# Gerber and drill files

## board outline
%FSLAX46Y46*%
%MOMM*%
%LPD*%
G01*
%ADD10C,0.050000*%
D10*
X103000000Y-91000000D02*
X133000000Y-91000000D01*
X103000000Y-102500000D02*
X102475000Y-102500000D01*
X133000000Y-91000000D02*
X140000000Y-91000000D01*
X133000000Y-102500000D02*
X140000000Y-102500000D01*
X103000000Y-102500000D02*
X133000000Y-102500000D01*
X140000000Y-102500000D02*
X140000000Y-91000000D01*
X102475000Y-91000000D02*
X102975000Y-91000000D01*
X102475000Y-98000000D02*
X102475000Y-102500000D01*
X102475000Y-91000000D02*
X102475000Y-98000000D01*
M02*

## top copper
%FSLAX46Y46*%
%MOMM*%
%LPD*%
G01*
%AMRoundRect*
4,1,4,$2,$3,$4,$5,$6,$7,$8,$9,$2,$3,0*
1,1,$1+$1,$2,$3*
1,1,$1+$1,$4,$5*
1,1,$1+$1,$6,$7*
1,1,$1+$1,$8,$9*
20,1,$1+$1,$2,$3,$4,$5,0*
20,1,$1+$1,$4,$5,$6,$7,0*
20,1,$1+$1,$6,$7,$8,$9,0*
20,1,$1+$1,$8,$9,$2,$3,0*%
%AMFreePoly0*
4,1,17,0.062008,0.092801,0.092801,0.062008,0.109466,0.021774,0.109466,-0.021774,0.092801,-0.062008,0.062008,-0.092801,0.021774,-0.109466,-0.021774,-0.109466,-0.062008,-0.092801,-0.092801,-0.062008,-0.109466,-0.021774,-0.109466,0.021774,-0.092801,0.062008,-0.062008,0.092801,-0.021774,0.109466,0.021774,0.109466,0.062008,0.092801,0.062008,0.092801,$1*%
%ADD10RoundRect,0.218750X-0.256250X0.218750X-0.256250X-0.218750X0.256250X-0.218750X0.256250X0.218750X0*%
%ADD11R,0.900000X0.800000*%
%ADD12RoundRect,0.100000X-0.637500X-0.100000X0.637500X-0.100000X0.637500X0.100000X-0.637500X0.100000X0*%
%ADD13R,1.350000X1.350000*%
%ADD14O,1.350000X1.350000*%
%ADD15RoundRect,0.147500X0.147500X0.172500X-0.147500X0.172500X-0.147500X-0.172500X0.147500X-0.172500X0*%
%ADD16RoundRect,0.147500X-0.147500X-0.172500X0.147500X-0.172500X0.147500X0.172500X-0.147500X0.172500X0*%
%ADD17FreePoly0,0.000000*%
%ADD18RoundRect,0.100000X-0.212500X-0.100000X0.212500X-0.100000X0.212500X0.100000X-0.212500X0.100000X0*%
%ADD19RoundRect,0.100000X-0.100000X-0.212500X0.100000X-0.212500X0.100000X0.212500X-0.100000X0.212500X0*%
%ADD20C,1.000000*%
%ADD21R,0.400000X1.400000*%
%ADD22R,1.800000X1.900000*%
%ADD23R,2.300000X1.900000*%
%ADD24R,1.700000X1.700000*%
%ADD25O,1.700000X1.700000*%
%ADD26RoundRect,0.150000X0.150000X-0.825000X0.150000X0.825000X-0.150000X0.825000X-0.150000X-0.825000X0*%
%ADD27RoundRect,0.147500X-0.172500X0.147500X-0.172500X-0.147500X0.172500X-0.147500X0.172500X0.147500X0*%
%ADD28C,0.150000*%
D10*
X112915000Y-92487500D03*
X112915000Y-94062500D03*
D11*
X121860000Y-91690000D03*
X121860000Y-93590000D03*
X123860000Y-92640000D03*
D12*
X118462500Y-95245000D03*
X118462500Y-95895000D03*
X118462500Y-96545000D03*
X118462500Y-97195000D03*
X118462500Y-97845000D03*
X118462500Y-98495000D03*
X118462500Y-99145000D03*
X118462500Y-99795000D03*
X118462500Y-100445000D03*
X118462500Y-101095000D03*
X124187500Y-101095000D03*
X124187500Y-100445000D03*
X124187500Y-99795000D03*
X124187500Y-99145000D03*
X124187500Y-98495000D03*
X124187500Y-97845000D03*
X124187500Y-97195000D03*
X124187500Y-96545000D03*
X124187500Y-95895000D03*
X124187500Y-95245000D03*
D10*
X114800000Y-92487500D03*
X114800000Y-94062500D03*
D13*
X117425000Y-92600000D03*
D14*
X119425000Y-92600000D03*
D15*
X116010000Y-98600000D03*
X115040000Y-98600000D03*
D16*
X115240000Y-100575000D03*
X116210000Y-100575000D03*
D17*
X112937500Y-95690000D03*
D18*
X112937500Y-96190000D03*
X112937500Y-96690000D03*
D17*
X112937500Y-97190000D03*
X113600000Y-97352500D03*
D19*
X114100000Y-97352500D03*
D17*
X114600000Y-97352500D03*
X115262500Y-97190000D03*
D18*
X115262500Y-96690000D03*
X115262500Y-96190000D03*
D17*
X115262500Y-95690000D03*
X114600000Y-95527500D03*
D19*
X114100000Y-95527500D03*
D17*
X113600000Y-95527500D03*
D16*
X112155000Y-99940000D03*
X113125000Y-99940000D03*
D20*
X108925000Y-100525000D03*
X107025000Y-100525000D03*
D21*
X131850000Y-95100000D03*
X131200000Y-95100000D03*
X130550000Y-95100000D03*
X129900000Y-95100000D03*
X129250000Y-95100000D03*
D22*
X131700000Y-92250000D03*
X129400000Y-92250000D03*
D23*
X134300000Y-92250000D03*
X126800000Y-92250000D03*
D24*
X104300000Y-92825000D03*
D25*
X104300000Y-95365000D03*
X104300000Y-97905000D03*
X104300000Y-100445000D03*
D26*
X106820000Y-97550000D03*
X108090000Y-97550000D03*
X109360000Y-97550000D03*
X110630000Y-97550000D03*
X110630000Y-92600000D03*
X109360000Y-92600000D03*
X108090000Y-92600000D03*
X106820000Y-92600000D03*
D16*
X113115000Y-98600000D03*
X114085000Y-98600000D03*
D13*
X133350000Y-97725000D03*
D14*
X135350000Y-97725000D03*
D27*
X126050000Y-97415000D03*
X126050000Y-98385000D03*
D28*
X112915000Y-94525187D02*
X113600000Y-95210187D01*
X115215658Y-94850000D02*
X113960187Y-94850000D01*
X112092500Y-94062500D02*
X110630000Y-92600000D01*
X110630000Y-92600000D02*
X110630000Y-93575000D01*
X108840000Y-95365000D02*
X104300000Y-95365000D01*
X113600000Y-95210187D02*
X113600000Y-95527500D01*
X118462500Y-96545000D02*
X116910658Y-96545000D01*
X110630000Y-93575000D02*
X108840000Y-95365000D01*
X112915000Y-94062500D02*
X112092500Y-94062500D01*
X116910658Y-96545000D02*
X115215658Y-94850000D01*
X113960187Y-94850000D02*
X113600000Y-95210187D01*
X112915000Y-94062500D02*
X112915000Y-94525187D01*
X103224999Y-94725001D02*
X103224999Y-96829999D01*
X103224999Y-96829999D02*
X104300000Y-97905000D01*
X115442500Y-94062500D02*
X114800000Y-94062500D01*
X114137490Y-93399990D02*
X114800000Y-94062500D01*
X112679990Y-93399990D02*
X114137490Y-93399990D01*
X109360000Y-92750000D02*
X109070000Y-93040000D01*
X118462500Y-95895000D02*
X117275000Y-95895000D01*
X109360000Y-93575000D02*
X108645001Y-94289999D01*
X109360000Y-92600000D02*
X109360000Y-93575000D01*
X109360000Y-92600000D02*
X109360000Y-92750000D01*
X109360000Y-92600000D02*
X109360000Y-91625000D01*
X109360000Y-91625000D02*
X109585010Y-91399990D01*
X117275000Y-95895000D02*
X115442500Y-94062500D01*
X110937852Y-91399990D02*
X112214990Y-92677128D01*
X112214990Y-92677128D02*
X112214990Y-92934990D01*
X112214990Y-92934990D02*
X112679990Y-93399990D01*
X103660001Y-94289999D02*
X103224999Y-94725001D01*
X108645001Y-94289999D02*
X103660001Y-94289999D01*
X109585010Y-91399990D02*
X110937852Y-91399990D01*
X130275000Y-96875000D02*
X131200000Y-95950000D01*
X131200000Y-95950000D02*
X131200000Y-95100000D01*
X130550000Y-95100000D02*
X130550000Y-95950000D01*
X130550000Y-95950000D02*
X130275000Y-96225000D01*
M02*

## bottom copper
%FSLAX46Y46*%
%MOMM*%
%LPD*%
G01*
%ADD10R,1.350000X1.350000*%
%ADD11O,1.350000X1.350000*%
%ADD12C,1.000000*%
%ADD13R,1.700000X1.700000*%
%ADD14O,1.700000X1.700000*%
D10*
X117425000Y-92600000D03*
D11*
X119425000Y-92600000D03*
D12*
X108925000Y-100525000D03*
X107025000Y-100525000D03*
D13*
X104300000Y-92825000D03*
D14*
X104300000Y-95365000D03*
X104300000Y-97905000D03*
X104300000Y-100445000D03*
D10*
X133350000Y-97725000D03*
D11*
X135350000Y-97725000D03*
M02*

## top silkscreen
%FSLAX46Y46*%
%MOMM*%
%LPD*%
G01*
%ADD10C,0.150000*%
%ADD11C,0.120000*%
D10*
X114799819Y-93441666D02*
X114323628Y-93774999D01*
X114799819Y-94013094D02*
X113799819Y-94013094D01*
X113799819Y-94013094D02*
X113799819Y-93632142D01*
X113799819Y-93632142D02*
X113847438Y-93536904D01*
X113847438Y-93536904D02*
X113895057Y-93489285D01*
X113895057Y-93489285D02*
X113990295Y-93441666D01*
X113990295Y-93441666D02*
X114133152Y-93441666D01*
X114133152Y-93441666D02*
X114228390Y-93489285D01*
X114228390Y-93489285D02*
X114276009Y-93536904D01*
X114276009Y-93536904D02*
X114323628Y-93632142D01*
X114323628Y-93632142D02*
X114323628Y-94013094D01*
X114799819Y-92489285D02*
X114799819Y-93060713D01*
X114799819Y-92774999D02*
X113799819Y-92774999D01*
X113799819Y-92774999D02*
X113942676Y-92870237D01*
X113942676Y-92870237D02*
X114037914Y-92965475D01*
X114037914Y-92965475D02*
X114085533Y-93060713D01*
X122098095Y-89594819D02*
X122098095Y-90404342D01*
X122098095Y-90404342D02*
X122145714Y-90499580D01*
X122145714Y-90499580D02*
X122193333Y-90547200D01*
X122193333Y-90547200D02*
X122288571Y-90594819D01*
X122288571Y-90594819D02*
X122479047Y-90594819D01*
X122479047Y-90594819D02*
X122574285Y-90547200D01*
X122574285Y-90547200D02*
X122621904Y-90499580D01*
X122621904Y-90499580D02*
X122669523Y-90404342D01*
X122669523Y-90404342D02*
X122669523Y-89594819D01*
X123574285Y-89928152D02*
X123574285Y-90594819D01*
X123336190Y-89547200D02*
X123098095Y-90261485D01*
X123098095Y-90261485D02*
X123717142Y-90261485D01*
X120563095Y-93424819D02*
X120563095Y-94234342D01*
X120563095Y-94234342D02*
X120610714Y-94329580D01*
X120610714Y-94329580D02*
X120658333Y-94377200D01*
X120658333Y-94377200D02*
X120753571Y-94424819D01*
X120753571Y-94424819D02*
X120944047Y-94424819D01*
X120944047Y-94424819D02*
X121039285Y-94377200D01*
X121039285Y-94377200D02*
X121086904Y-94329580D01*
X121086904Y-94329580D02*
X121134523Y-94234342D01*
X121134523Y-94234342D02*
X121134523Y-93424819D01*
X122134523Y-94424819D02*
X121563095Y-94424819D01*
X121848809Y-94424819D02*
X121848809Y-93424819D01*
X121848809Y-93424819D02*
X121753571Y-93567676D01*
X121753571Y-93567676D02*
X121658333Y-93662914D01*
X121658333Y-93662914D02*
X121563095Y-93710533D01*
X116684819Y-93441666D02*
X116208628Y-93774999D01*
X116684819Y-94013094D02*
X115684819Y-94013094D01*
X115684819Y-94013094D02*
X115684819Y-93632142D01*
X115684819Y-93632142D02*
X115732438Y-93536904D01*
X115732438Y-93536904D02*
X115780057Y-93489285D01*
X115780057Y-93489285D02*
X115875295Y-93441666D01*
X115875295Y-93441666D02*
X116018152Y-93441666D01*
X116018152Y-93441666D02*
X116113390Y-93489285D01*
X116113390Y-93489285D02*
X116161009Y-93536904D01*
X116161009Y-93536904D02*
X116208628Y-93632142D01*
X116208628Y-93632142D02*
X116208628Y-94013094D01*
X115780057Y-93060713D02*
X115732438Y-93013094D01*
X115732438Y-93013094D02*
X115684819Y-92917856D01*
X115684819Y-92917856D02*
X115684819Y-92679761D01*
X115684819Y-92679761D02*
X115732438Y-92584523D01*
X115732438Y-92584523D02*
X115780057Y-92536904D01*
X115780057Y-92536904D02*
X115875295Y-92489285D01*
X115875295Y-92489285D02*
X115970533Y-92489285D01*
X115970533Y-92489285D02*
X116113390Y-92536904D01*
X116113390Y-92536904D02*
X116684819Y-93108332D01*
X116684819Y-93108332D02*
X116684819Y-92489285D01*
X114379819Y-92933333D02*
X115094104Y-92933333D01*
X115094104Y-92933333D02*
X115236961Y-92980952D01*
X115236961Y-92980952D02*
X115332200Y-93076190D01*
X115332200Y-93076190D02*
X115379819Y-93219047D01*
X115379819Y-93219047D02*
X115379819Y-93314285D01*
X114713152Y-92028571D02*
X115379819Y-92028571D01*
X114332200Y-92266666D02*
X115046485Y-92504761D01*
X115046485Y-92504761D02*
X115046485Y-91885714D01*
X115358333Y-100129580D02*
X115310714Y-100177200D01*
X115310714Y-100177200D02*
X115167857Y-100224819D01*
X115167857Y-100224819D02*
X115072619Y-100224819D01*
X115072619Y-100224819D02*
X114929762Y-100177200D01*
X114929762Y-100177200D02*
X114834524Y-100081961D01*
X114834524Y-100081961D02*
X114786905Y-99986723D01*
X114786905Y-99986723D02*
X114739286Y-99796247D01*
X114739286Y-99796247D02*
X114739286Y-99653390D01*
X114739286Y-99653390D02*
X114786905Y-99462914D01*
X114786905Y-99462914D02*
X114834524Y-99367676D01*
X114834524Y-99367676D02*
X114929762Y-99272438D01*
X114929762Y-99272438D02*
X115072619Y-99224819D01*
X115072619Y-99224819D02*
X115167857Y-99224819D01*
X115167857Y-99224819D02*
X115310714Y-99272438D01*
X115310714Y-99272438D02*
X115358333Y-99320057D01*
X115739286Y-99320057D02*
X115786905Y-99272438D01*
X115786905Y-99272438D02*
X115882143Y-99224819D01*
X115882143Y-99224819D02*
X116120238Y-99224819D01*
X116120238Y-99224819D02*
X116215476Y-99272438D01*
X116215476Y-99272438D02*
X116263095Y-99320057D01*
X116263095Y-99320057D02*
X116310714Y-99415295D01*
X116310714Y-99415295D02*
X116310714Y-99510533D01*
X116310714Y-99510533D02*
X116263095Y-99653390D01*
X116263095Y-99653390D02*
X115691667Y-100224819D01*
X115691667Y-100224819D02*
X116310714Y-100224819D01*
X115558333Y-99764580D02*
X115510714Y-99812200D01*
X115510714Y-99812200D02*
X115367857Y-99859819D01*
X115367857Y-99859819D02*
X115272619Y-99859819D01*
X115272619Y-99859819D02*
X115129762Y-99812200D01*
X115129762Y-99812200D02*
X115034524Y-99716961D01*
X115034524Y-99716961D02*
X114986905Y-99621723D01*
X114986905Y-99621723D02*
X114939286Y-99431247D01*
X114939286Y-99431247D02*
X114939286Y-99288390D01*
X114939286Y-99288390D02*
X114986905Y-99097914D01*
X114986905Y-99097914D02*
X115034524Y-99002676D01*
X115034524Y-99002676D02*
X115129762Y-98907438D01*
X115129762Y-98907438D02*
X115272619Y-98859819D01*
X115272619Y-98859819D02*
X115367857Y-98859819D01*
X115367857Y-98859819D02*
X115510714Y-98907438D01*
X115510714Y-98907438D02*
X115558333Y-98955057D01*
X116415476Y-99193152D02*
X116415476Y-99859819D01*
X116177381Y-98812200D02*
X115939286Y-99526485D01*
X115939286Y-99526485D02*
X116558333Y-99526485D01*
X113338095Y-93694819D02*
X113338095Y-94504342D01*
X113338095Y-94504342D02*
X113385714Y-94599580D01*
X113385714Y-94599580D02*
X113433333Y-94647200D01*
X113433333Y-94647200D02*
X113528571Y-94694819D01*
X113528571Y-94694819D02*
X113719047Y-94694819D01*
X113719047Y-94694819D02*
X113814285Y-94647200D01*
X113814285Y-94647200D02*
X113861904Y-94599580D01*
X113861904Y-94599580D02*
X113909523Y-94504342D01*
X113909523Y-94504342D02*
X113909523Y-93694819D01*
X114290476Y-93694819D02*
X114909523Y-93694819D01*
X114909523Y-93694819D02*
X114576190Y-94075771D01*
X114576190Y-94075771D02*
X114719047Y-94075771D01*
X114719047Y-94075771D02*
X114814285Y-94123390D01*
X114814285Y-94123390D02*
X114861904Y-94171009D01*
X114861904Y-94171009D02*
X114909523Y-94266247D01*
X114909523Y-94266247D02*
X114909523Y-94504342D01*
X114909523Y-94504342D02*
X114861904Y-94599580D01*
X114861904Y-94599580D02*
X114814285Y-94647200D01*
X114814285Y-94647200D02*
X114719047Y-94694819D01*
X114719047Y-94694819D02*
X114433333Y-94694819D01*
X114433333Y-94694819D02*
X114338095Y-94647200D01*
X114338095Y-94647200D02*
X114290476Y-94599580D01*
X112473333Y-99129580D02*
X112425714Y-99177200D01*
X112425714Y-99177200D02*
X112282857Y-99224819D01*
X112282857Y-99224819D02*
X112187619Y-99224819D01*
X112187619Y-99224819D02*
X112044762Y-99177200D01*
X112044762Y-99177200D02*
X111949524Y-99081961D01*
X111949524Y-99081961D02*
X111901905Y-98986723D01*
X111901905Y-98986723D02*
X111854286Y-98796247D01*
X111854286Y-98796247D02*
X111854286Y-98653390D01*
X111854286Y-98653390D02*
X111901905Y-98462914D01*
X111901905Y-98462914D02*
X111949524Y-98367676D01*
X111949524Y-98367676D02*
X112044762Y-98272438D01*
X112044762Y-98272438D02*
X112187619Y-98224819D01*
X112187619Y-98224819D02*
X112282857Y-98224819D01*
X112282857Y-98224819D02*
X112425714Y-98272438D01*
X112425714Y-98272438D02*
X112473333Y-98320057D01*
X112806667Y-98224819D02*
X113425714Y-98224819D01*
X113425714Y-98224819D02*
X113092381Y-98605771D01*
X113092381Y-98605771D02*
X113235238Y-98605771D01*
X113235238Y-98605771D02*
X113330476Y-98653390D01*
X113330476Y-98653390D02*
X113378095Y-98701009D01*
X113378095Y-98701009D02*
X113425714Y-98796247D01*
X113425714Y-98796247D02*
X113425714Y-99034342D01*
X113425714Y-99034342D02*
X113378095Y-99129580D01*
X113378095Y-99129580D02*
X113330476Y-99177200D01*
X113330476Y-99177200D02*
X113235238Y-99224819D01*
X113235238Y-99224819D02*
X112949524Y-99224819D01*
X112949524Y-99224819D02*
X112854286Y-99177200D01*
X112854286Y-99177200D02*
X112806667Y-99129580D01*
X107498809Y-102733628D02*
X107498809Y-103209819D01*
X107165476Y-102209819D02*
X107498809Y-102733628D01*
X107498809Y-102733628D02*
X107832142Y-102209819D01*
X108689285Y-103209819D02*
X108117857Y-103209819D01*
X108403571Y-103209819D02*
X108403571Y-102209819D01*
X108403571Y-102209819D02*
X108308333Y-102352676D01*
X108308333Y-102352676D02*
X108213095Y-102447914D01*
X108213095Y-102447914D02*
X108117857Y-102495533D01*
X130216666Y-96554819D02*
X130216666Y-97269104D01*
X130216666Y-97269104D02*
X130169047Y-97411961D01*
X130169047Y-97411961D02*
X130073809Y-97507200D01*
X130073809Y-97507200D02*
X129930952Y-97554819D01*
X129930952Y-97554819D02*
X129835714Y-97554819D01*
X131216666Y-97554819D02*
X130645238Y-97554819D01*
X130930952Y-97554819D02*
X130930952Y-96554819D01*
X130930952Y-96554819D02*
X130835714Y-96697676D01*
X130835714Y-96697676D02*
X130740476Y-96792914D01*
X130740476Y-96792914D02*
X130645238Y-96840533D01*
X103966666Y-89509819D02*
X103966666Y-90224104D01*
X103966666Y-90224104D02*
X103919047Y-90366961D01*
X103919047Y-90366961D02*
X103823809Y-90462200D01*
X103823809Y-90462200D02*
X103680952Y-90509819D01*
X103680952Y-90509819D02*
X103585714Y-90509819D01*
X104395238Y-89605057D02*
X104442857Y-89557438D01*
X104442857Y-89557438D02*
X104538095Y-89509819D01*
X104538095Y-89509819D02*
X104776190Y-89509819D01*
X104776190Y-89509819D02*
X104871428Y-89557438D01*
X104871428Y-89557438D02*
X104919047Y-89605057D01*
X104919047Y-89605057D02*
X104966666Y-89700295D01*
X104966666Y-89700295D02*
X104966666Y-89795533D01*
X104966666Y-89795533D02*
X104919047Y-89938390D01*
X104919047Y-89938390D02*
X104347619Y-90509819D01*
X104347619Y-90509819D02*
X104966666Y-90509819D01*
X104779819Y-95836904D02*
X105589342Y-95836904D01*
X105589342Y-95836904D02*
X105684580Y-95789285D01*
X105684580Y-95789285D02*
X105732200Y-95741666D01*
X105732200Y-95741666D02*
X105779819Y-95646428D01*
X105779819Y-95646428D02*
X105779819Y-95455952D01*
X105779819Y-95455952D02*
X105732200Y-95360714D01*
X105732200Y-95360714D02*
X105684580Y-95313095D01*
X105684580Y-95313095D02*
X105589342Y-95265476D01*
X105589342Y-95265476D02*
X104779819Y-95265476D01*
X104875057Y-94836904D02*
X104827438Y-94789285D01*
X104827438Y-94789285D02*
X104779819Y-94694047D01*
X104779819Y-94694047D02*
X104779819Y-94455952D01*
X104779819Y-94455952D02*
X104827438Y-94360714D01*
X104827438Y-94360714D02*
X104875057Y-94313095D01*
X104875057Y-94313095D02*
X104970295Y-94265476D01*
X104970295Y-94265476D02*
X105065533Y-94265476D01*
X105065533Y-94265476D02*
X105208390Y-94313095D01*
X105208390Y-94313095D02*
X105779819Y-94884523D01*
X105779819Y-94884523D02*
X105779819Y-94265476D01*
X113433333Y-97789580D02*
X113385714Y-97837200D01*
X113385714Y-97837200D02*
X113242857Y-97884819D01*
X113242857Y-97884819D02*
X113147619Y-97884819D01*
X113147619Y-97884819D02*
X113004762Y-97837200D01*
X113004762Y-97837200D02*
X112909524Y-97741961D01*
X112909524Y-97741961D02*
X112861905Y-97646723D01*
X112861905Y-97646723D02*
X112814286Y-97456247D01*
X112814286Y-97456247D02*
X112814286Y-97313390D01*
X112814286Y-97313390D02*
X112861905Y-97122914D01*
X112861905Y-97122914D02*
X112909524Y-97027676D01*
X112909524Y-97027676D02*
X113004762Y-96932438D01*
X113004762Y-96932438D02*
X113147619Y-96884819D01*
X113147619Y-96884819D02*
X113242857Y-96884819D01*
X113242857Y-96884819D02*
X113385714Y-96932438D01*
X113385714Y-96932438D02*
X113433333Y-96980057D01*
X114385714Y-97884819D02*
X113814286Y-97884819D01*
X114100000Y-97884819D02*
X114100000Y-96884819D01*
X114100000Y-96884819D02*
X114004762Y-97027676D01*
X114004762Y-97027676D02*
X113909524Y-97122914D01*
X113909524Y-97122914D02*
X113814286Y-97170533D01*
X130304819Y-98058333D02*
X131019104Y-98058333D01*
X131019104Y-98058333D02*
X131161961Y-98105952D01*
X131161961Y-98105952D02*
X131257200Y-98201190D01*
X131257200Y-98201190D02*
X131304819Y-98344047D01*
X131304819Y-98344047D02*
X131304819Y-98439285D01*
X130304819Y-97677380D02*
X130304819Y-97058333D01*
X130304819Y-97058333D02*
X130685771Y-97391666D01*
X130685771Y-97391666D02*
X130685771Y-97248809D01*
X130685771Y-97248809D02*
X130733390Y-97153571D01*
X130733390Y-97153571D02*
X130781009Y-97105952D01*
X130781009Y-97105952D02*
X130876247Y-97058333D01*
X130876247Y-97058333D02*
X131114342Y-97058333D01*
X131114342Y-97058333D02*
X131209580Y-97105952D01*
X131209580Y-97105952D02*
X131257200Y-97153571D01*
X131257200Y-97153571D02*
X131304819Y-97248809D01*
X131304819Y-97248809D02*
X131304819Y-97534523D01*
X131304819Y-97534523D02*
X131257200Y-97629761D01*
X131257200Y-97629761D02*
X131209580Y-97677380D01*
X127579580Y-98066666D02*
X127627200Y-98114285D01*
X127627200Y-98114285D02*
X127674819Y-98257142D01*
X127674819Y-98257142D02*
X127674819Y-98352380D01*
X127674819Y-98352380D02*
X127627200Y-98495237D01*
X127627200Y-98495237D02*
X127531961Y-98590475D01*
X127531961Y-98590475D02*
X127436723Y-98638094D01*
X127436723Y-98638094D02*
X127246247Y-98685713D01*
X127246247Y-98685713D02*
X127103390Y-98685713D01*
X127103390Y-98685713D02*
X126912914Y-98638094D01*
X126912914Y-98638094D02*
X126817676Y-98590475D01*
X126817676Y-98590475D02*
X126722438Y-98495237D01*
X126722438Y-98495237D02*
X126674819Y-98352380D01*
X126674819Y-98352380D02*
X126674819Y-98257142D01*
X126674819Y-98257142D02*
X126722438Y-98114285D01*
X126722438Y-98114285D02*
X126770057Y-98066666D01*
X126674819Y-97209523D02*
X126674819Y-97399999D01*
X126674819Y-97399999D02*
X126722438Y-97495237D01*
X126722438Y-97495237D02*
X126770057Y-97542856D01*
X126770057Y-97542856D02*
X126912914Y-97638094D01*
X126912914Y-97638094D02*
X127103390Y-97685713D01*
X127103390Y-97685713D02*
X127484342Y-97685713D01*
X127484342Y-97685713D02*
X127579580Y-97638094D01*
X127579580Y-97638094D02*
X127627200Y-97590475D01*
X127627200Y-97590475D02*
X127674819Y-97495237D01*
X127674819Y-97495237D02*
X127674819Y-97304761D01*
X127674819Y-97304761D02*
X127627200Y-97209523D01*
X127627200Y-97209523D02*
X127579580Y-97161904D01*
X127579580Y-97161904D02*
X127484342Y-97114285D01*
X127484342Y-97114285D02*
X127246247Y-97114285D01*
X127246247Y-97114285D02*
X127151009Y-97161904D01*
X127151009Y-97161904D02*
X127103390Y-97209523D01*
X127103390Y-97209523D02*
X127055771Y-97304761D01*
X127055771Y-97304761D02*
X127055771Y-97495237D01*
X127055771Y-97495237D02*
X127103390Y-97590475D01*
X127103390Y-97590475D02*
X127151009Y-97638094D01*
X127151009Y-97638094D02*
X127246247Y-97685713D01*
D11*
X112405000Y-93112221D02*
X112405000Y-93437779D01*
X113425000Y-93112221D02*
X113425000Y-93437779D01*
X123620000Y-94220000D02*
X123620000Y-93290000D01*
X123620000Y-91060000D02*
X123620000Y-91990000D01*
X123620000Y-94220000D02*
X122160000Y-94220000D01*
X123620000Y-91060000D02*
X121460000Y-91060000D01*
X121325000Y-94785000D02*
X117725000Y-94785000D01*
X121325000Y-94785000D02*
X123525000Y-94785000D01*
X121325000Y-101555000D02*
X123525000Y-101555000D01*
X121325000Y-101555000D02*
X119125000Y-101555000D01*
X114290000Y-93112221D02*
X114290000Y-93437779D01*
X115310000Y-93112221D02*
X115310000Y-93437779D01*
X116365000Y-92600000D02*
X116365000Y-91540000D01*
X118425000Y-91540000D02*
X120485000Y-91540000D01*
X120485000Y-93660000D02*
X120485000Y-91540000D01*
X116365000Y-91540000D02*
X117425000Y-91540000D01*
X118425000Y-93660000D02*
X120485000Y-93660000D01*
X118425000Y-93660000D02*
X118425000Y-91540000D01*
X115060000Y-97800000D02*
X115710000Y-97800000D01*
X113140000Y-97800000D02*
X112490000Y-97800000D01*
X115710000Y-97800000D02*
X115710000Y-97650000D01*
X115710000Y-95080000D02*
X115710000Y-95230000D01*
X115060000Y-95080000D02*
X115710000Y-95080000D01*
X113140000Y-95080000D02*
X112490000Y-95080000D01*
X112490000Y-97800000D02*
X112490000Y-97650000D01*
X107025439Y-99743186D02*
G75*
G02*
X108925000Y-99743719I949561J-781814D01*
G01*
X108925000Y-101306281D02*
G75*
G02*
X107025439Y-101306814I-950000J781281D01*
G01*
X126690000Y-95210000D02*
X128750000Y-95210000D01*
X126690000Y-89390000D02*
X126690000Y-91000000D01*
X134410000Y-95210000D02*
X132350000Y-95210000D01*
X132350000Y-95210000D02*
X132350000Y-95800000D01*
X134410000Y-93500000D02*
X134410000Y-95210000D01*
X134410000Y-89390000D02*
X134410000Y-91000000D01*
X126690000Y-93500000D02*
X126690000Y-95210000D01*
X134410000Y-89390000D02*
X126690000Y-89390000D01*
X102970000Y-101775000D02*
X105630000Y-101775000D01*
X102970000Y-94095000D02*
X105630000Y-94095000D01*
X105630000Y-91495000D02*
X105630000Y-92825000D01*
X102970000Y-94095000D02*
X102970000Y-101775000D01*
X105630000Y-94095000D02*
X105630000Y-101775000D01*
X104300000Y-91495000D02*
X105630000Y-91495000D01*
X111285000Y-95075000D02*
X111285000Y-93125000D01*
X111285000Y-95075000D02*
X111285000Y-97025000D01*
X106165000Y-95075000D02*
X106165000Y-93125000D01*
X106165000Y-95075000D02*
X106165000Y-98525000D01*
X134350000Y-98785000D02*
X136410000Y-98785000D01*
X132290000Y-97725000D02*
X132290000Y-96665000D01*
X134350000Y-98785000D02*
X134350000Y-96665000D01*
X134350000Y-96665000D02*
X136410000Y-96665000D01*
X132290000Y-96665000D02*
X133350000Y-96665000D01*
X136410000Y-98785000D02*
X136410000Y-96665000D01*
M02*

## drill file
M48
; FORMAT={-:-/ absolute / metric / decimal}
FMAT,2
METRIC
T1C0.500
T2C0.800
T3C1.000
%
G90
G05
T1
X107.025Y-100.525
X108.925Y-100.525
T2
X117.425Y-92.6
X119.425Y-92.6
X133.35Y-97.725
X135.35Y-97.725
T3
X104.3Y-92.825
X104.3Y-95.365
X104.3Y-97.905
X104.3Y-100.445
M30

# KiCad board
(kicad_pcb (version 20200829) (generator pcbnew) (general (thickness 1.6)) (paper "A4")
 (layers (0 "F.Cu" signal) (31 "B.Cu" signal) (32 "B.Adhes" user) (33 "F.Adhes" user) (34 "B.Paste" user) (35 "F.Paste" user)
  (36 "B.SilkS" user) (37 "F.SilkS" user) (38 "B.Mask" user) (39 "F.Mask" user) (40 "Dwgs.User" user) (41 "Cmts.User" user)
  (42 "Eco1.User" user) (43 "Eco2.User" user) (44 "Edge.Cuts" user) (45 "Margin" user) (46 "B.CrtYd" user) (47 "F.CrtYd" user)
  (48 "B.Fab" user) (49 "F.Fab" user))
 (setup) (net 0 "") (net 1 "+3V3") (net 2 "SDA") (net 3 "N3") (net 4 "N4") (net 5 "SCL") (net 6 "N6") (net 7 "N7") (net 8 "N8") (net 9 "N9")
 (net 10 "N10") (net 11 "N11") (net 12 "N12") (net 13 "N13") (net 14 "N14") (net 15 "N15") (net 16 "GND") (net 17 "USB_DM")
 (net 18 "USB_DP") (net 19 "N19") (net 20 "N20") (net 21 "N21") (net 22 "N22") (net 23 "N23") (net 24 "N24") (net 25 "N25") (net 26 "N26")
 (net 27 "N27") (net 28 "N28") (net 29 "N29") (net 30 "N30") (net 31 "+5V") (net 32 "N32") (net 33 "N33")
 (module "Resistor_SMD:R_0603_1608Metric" (layer "F.Cu") (at 112.915 93.275 -90)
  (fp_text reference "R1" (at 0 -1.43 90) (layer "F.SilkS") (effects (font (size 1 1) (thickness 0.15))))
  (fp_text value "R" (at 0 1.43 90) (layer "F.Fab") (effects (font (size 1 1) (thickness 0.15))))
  (fp_line (start -0.162779 0.51) (end 0.162779 0.51) (layer "F.SilkS") (width 0.12))
  (fp_line (start -0.162779 -0.51) (end 0.162779 -0.51) (layer "F.SilkS") (width 0.12))
  (pad "1" smd roundrect (at -0.7875 0 270) (size 0.875 0.95) (layers "F.Cu" "F.Paste" "F.Mask") (roundrect_rratio 0.25) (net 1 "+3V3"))
  (pad "2" smd roundrect (at 0.7875 0 270) (size 0.875 0.95) (layers "F.Cu" "F.Paste" "F.Mask") (roundrect_rratio 0.25) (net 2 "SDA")))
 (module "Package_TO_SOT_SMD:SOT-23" (layer "F.Cu") (at 122.86 92.64)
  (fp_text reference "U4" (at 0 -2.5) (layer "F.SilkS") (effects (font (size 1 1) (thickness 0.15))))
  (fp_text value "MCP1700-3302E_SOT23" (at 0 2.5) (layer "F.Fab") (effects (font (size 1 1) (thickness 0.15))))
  (fp_line (start 0.76 1.58) (end 0.76 0.65) (layer "F.SilkS") (width 0.12))
  (fp_line (start 0.76 -1.58) (end 0.76 -0.65) (layer "F.SilkS") (width 0.12))
  (fp_line (start 0.76 1.58) (end -0.7 1.58) (layer "F.SilkS") (width 0.12))
  (fp_line (start 0.76 -1.58) (end -1.4 -1.58) (layer "F.SilkS") (width 0.12))
  (pad "1" smd rect (at -1 -0.95) (size 0.9 0.8) (layers "F.Cu" "F.Paste" "F.Mask") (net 1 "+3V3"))
  (pad "2" smd rect (at -1 0.95) (size 0.9 0.8) (layers "F.Cu" "F.Paste" "F.Mask") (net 1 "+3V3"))
  (pad "3" smd rect (at 1 0) (size 0.9 0.8) (layers "F.Cu" "F.Paste" "F.Mask") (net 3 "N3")))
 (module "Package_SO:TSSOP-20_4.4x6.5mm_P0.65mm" (layer "F.Cu") (at 121.325 98.17)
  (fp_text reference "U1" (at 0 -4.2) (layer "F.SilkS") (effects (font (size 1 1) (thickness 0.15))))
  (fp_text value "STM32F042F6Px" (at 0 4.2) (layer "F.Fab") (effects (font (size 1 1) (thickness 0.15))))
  (fp_line (start 0 -3.385) (end -3.6 -3.385) (layer "F.SilkS") (width 0.12))
  (fp_line (start 0 -3.385) (end 2.2 -3.385) (layer "F.SilkS") (width 0.12))
  (fp_line (start 0 3.385) (end 2.2 3.385) (layer "F.SilkS") (width 0.12))
  (fp_line (start 0 3.385) (end -2.2 3.385) (layer "F.SilkS") (width 0.12))
  (pad "1" smd roundrect (at -2.8625 -2.925) (size 1.475 0.4) (layers "F.Cu" "F.Paste" "F.Mask") (roundrect_rratio 0.25) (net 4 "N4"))
  (pad "2" smd roundrect (at -2.8625 -2.275) (size 1.475 0.4) (layers "F.Cu" "F.Paste" "F.Mask") (roundrect_rratio 0.25) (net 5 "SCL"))
  (pad "3" smd roundrect (at -2.8625 -1.625) (size 1.475 0.4) (layers "F.Cu" "F.Paste" "F.Mask") (roundrect_rratio 0.25) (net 2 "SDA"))
  (pad "4" smd roundrect (at -2.8625 -0.975) (size 1.475 0.4) (layers "F.Cu" "F.Paste" "F.Mask") (roundrect_rratio 0.25) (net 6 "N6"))
  (pad "5" smd roundrect (at -2.8625 -0.325) (size 1.475 0.4) (layers "F.Cu" "F.Paste" "F.Mask") (roundrect_rratio 0.25) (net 1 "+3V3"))
  (pad "6" smd roundrect (at -2.8625 0.325) (size 1.475 0.4) (layers "F.Cu" "F.Paste" "F.Mask") (roundrect_rratio 0.25) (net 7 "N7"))
  (pad "7" smd roundrect (at -2.8625 0.975) (size 1.475 0.4) (layers "F.Cu" "F.Paste" "F.Mask") (roundrect_rratio 0.25) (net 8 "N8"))
  (pad "8" smd roundrect (at -2.8625 1.625) (size 1.475 0.4) (layers "F.Cu" "F.Paste" "F.Mask") (roundrect_rratio 0.25) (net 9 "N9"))
  (pad "9" smd roundrect (at -2.8625 2.275) (size 1.475 0.4) (layers "F.Cu" "F.Paste" "F.Mask") (roundrect_rratio 0.25) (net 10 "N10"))
  (pad "10" smd roundrect (at -2.8625 2.925) (size 1.475 0.4) (layers "F.Cu" "F.Paste" "F.Mask") (roundrect_rratio 0.25) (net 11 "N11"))
  (pad "11" smd roundrect (at 2.8625 2.925) (size 1.475 0.4) (layers "F.Cu" "F.Paste" "F.Mask") (roundrect_rratio 0.25) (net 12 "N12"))
  (pad "12" smd roundrect (at 2.8625 2.275) (size 1.475 0.4) (layers "F.Cu" "F.Paste" "F.Mask") (roundrect_rratio 0.25) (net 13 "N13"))
  (pad "13" smd roundrect (at 2.8625 1.625) (size 1.475 0.4) (layers "F.Cu" "F.Paste" "F.Mask") (roundrect_rratio 0.25) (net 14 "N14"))
  (pad "14" smd roundrect (at 2.8625 0.975) (size 1.475 0.4) (layers "F.Cu" "F.Paste" "F.Mask") (roundrect_rratio 0.25) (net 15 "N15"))
  (pad "15" smd roundrect (at 2.8625 0.325) (size 1.475 0.4) (layers "F.Cu" "F.Paste" "F.Mask") (roundrect_rratio 0.25) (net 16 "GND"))
  (pad "16" smd roundrect (at 2.8625 -0.325) (size 1.475 0.4) (layers "F.Cu" "F.Paste" "F.Mask") (roundrect_rratio 0.25) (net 1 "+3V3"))
  (pad "17" smd roundrect (at 2.8625 -0.975) (size 1.475 0.4) (layers "F.Cu" "F.Paste" "F.Mask") (roundrect_rratio 0.25) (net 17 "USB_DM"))
  (pad "18" smd roundrect (at 2.8625 -1.625) (size 1.475 0.4) (layers "F.Cu" "F.Paste" "F.Mask") (roundrect_rratio 0.25) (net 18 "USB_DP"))
  (pad "19" smd roundrect (at 2.8625 -2.275) (size 1.475 0.4) (layers "F.Cu" "F.Paste" "F.Mask") (roundrect_rratio 0.25) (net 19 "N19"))
  (pad "20" smd roundrect (at 2.8625 -2.925) (size 1.475 0.4) (layers "F.Cu" "F.Paste" "F.Mask") (roundrect_rratio 0.25) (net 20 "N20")))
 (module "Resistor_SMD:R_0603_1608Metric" (layer "F.Cu") (at 114.8 93.275 -90)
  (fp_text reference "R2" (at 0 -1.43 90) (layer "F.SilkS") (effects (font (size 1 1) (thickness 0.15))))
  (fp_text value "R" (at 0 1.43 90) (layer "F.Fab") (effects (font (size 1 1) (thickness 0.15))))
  (fp_line (start -0.162779 0.51) (end 0.162779 0.51) (layer "F.SilkS") (width 0.12))
  (fp_line (start -0.162779 -0.51) (end 0.162779 -0.51) (layer "F.SilkS") (width 0.12))
  (pad "1" smd roundrect (at -0.7875 0 270) (size 0.875 0.95) (layers "F.Cu" "F.Paste" "F.Mask") (roundrect_rratio 0.25) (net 1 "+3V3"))
  (pad "2" smd roundrect (at 0.7875 0 270) (size 0.875 0.95) (layers "F.Cu" "F.Paste" "F.Mask") (roundrect_rratio 0.25) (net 5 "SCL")))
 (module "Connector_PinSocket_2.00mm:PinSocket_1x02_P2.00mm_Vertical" (layer "F.Cu") (at 117.425 92.6 90)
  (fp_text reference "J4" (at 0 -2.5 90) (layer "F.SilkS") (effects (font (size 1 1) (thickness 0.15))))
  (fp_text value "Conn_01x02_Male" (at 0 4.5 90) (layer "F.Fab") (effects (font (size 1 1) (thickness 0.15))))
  (fp_line (start 0 -1.06) (end 1.06 -1.06) (layer "F.SilkS") (width 0.12))
  (fp_line (start 1.06 1) (end 1.06 3.06) (layer "F.SilkS") (width 0.12))
  (fp_line (start -1.06 3.06) (end 1.06 3.06) (layer "F.SilkS") (width 0.12))
  (fp_line (start 1.06 -1.06) (end 1.06 0) (layer "F.SilkS") (width 0.12))
  (fp_line (start -1.06 1) (end -1.06 3.06) (layer "F.SilkS") (width 0.12))
  (fp_line (start -1.06 1) (end 1.06 1) (layer "F.SilkS") (width 0.12))
  (pad "1" thru_hole rect (at 0 0 90) (size 1.35 1.35) (drill 0.8) (layers *.Cu *.Mask) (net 3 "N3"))
  (pad "2" thru_hole oval (at 0 2 90) (size 1.35 1.35) (drill 0.8) (layers *.Cu *.Mask) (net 1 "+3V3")))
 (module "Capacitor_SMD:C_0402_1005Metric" (layer "F.Cu") (at 115.525 98.6 180)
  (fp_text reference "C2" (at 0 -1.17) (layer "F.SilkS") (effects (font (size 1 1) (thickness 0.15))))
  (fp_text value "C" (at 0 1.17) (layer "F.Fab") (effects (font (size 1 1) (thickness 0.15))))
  (pad "1" smd roundrect (at -0.485 0 180) (size 0.59 0.64) (layers "F.Cu" "F.Paste" "F.Mask") (roundrect_rratio 0.25) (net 1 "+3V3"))
  (pad "2" smd roundrect (at 0.485 0 180) (size 0.59 0.64) (layers "F.Cu" "F.Paste" "F.Mask") (roundrect_rratio 0.25) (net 16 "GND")))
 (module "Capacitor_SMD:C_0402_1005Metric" (layer "F.Cu") (at 115.725 100.575)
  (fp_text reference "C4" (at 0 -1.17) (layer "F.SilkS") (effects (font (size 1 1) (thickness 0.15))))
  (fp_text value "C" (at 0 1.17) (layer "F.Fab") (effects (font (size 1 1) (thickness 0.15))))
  (pad "1" smd roundrect (at -0.485 0) (size 0.59 0.64) (layers "F.Cu" "F.Paste" "F.Mask") (roundrect_rratio 0.25) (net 16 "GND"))
  (pad "2" smd roundrect (at 0.485 0) (size 0.59 0.64) (layers "F.Cu" "F.Paste" "F.Mask") (roundrect_rratio 0.25) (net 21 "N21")))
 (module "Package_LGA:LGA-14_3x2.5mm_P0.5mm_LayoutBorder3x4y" (layer "F.Cu") (at 114.1 96.44)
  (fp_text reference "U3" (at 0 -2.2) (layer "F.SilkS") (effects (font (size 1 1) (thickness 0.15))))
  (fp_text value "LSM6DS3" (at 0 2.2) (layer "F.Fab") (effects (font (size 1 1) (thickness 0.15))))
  (fp_line (start 0.96 1.36) (end 1.61 1.36) (layer "F.SilkS") (width 0.12))
  (fp_line (start -0.96 1.36) (end -1.61 1.36) (layer "F.SilkS") (width 0.12))
  (fp_line (start 1.61 1.36) (end 1.61 1.21) (layer "F.SilkS") (width 0.12))
  (fp_line (start 1.61 -1.36) (end 1.61 -1.21) (layer "F.SilkS") (width 0.12))
  (fp_line (start 0.96 -1.36) (end 1.61 -1.36) (layer "F.SilkS") (width 0.12))
  (fp_line (start -0.96 -1.36) (end -1.61 -1.36) (layer "F.SilkS") (width 0.12))
  (fp_line (start -1.61 1.36) (end -1.61 1.21) (layer "F.SilkS") (width 0.12))
  (pad "1" smd custom (at -1.1625 -0.75) (size 0.223223 0.223223) (layers "F.Cu" "F.Paste" "F.Mask") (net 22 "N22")
   (options (clearance outline) (anchor circle)) (primitives))
  (pad "2" smd roundrect (at -1.1625 -0.25) (size 0.625 0.4) (layers "F.Cu" "F.Paste" "F.Mask") (roundrect_rratio 0.25) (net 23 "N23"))
  (pad "3" smd roundrect (at -1.1625 0.25) (size 0.625 0.4) (layers "F.Cu" "F.Paste" "F.Mask") (roundrect_rratio 0.25) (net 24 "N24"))
  (pad "4" smd custom (at -1.1625 0.75) (size 0.223223 0.223223) (layers "F.Cu" "F.Paste" "F.Mask") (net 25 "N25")
   (options (clearance outline) (anchor circle)) (primitives))
  (pad "5" smd custom (at -0.5 0.9125) (size 0.223223 0.223223) (layers "F.Cu" "F.Paste" "F.Mask") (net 1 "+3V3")
   (options (clearance outline) (anchor circle)) (primitives))
  (pad "6" smd roundrect (at 0 0.9125) (size 0.4 0.625) (layers "F.Cu" "F.Paste" "F.Mask") (roundrect_rratio 0.25) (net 16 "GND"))
  (pad "7" smd custom (at 0.5 0.9125) (size 0.223223 0.223223) (layers "F.Cu" "F.Paste" "F.Mask") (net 16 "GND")
   (options (clearance outline) (anchor circle)) (primitives))
  (pad "8" smd custom (at 1.1625 0.75) (size 0.223223 0.223223) (layers "F.Cu" "F.Paste" "F.Mask") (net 1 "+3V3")
   (options (clearance outline) (anchor circle)) (primitives))
  (pad "9" smd roundrect (at 1.1625 0.25) (size 0.625 0.4) (layers "F.Cu" "F.Paste" "F.Mask") (roundrect_rratio 0.25) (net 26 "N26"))
  (pad "10" smd roundrect (at 1.1625 -0.25) (size 0.625 0.4) (layers "F.Cu" "F.Paste" "F.Mask") (roundrect_rratio 0.25) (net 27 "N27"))
  (pad "11" smd custom (at 1.1625 -0.75) (size 0.223223 0.223223) (layers "F.Cu" "F.Paste" "F.Mask") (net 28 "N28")
   (options (clearance outline) (anchor circle)) (primitives))
  (pad "12" smd custom (at 0.5 -0.9125) (size 0.223223 0.223223) (layers "F.Cu" "F.Paste" "F.Mask") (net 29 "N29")
   (options (clearance outline) (anchor circle)) (primitives))
  (pad "13" smd roundrect (at 0 -0.9125) (size 0.4 0.625) (layers "F.Cu" "F.Paste" "F.Mask") (roundrect_rratio 0.25) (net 5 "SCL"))
  (pad "14" smd custom (at -0.5 -0.9125) (size 0.223223 0.223223) (layers "F.Cu" "F.Paste" "F.Mask") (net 2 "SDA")
   (options (clearance outline) (anchor circle)) (primitives)))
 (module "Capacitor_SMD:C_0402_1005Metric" (layer "F.Cu") (at 112.64 99.94)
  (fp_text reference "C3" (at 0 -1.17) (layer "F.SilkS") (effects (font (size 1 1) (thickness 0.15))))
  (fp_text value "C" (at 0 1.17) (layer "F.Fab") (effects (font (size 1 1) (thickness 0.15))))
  (pad "1" smd roundrect (at -0.485 0) (size 0.59 0.64) (layers "F.Cu" "F.Paste" "F.Mask") (roundrect_rratio 0.25) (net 16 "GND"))
  (pad "2" smd roundrect (at 0.485 0) (size 0.59 0.64) (layers "F.Cu" "F.Paste" "F.Mask") (roundrect_rratio 0.25) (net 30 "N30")))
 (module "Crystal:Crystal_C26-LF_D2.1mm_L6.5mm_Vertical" (layer "F.Cu") (at 108.925 100.525 180)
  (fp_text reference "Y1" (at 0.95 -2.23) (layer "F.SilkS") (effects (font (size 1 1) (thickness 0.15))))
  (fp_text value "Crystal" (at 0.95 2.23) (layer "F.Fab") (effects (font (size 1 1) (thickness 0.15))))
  (fp_arc (start 0.95 0) (end 0 0.781281) (angle -101.1) (layer "F.SilkS") (width 0.12))
  (fp_arc (start 0.95 0) (end 0 -0.781281) (angle 101.1) (layer "F.SilkS") (width 0.12))
  (pad "1" thru_hole circle (at 0 0 180) (size 1 1) (drill 0.5) (layers *.Cu *.Mask) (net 21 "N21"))
  (pad "2" thru_hole circle (at 1.9 0 180) (size 1 1) (drill 0.5) (layers *.Cu *.Mask) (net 30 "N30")))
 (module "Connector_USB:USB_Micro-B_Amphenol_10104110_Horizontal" (layer "F.Cu") (at 130.55 93.55 180)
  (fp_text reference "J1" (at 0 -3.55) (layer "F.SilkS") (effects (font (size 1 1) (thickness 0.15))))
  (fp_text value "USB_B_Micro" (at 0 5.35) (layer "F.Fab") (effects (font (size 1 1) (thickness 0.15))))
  (fp_line (start 3.86 -1.66) (end 1.8 -1.66) (layer "F.SilkS") (width 0.12))
  (fp_line (start 3.86 4.16) (end 3.86 2.55) (layer "F.SilkS") (width 0.12))
  (fp_line (start -3.86 -1.66) (end -1.8 -1.66) (layer "F.SilkS") (width 0.12))
  (fp_line (start -1.8 -1.66) (end -1.8 -2.25) (layer "F.SilkS") (width 0.12))
  (fp_line (start -3.86 0.05) (end -3.86 -1.66) (layer "F.SilkS") (width 0.12))
  (fp_line (start -3.86 4.16) (end -3.86 2.55) (layer "F.SilkS") (width 0.12))
  (fp_line (start 3.86 0.05) (end 3.86 -1.66) (layer "F.SilkS") (width 0.12))
  (fp_line (start -3.86 4.16) (end 3.86 4.16) (layer "F.SilkS") (width 0.12))
  (pad "1" smd rect (at -1.3 -1.55 180) (size 0.4 1.4) (layers "F.Cu" "F.Paste" "F.Mask") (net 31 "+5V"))
  (pad "2" smd rect (at -0.65 -1.55 180) (size 0.4 1.4) (layers "F.Cu" "F.Paste" "F.Mask") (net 17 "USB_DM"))
  (pad "3" smd rect (at 0 -1.55 180) (size 0.4 1.4) (layers "F.Cu" "F.Paste" "F.Mask") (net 18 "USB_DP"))
  (pad "4" smd rect (at 0.65 -1.55 180) (size 0.4 1.4) (layers "F.Cu" "F.Paste" "F.Mask") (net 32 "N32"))
  (pad "5" smd rect (at 1.3 -1.55 180) (size 0.4 1.4) (layers "F.Cu" "F.Paste" "F.Mask") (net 16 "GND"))
  (pad "6" smd rect (at -1.15 1.3 180) (size 1.8 1.9) (layers "F.Cu" "F.Paste" "F.Mask") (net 16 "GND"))
  (pad "6" smd rect (at 1.15 1.3 180) (size 1.8 1.9) (layers "F.Cu" "F.Paste" "F.Mask") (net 16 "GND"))
  (pad "6" smd rect (at -3.75 1.3 180) (size 2.3 1.9) (layers "F.Cu" "F.Paste" "F.Mask") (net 16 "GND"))
  (pad "6" smd rect (at 3.75 1.3 180) (size 2.3 1.9) (layers "F.Cu" "F.Paste" "F.Mask") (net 16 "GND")))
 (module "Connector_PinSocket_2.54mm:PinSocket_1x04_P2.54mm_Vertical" (layer "F.Cu") (at 104.3 92.825)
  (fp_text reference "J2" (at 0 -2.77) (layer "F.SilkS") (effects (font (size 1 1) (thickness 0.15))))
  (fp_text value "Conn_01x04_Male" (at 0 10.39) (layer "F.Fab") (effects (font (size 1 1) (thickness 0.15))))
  (fp_line (start -1.33 8.95) (end 1.33 8.95) (layer "F.SilkS") (width 0.12))
  (fp_line (start -1.33 1.27) (end 1.33 1.27) (layer "F.SilkS") (width 0.12))
  (fp_line (start 1.33 -1.33) (end 1.33 0) (layer "F.SilkS") (width 0.12))
  (fp_line (start -1.33 1.27) (end -1.33 8.95) (layer "F.SilkS") (width 0.12))
  (fp_line (start 1.33 1.27) (end 1.33 8.95) (layer "F.SilkS") (width 0.12))
  (fp_line (start 0 -1.33) (end 1.33 -1.33) (layer "F.SilkS") (width 0.12))
  (pad "1" thru_hole rect (at 0 0) (size 1.7 1.7) (drill 1) (layers *.Cu *.Mask) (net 1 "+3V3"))
  (pad "2" thru_hole oval (at 0 2.54) (size 1.7 1.7) (drill 1) (layers *.Cu *.Mask) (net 2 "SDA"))
  (pad "3" thru_hole oval (at 0 5.08) (size 1.7 1.7) (drill 1) (layers *.Cu *.Mask) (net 5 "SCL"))
  (pad "4" thru_hole oval (at 0 7.62) (size 1.7 1.7) (drill 1) (layers *.Cu *.Mask) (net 16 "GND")))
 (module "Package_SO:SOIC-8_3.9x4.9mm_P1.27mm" (layer "F.Cu") (at 108.725 95.075 90)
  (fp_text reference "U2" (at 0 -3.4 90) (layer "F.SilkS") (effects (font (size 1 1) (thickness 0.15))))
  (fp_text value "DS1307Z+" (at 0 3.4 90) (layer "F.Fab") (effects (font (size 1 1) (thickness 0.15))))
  (fp_line (start 0 2.56) (end 1.95 2.56) (layer "F.SilkS") (width 0.12))
  (fp_line (start 0 2.56) (end -1.95 2.56) (layer "F.SilkS") (width 0.12))
  (fp_line (start 0 -2.56) (end 1.95 -2.56) (layer "F.SilkS") (width 0.12))
  (fp_line (start 0 -2.56) (end -3.45 -2.56) (layer "F.SilkS") (width 0.12))
  (pad "1" smd roundrect (at -2.475 -1.905 90) (size 1.95 0.6) (layers "F.Cu" "F.Paste" "F.Mask") (roundrect_rratio 0.25) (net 30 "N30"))
  (pad "2" smd roundrect (at -2.475 -0.635 90) (size 1.95 0.6) (layers "F.Cu" "F.Paste" "F.Mask") (roundrect_rratio 0.25) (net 21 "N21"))
  (pad "3" smd roundrect (at -2.475 0.635 90) (size 1.95 0.6) (layers "F.Cu" "F.Paste" "F.Mask") (roundrect_rratio 0.25) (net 1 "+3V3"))
  (pad "4" smd roundrect (at -2.475 1.905 90) (size 1.95 0.6) (layers "F.Cu" "F.Paste" "F.Mask") (roundrect_rratio 0.25) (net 16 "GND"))
  (pad "5" smd roundrect (at 2.475 1.905 90) (size 1.95 0.6) (layers "F.Cu" "F.Paste" "F.Mask") (roundrect_rratio 0.25) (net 2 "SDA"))
  (pad "6" smd roundrect (at 2.475 0.635 90) (size 1.95 0.6) (layers "F.Cu" "F.Paste" "F.Mask") (roundrect_rratio 0.25) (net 5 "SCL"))
  (pad "7" smd roundrect (at 2.475 -0.635 90) (size 1.95 0.6) (layers "F.Cu" "F.Paste" "F.Mask") (roundrect_rratio 0.25) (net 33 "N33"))
  (pad "8" smd roundrect (at 2.475 -1.905 90) (size 1.95 0.6) (layers "F.Cu" "F.Paste" "F.Mask") (roundrect_rratio 0.25) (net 1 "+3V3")))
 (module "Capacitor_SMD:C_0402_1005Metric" (layer "F.Cu") (at 113.6 98.6)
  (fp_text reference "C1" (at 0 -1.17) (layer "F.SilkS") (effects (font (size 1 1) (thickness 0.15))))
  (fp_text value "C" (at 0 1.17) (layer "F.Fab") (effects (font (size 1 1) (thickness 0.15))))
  (pad "1" smd roundrect (at -0.485 0) (size 0.59 0.64) (layers "F.Cu" "F.Paste" "F.Mask") (roundrect_rratio 0.25) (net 1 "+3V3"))
  (pad "2" smd roundrect (at 0.485 0) (size 0.59 0.64) (layers "F.Cu" "F.Paste" "F.Mask") (roundrect_rratio 0.25) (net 16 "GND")))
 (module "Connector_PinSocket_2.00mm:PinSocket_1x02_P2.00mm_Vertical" (layer "F.Cu") (at 133.35 97.725 90)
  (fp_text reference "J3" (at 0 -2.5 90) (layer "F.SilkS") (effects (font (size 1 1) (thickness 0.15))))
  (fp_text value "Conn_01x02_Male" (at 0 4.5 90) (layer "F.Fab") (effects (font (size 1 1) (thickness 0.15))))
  (fp_line (start -1.06 1) (end -1.06 3.06) (layer "F.SilkS") (width 0.12))
  (fp_line (start 0 -1.06) (end 1.06 -1.06) (layer "F.SilkS") (width 0.12))
  (fp_line (start -1.06 1) (end 1.06 1) (layer "F.SilkS") (width 0.12))
  (fp_line (start 1.06 1) (end 1.06 3.06) (layer "F.SilkS") (width 0.12))
  (fp_line (start 1.06 -1.06) (end 1.06 0) (layer "F.SilkS") (width 0.12))
  (fp_line (start -1.06 3.06) (end 1.06 3.06) (layer "F.SilkS") (width 0.12))
  (pad "1" thru_hole rect (at 0 0 90) (size 1.35 1.35) (drill 0.8) (layers *.Cu *.Mask) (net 31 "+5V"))
  (pad "2" thru_hole oval (at 0 2 90) (size 1.35 1.35) (drill 0.8) (layers *.Cu *.Mask) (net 16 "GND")))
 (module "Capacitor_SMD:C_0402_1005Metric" (layer "F.Cu") (at 126.05 97.9 -90)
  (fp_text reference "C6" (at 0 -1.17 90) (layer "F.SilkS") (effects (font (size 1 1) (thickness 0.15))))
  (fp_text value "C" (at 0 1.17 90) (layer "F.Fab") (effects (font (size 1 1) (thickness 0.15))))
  (pad "1" smd roundrect (at -0.485 0 270) (size 0.59 0.64) (layers "F.Cu" "F.Paste" "F.Mask") (roundrect_rratio 0.25) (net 1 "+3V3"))
  (pad "2" smd roundrect (at 0.485 0 270) (size 0.59 0.64) (layers "F.Cu" "F.Paste" "F.Mask") (roundrect_rratio 0.25) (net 16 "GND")))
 (gr_line (start 103 91) (end 133 91) (layer "Edge.Cuts") (width 0.05))
 (gr_line (start 103 102.5) (end 102.475 102.5) (layer "Edge.Cuts") (width 0.05))
 (gr_line (start 133 91) (end 140 91) (layer "Edge.Cuts") (width 0.05))
 (gr_line (start 133 102.5) (end 140 102.5) (layer "Edge.Cuts") (width 0.05))
 (gr_line (start 103 102.5) (end 133 102.5) (layer "Edge.Cuts") (width 0.05))
 (gr_line (start 140 102.5) (end 140 91) (layer "Edge.Cuts") (width 0.05))
 (gr_line (start 102.475 91) (end 102.975 91) (layer "Edge.Cuts") (width 0.05))
 (gr_line (start 102.475 98) (end 102.475 102.5) (layer "Edge.Cuts") (width 0.05))
 (gr_line (start 102.475 91) (end 102.475 98) (layer "Edge.Cuts") (width 0.05))
 (segment (start 112.915 94.525187) (end 113.6 95.210187) (width 0.15) (layer "F.Cu") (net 2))
 (segment (start 115.215658 94.85) (end 113.960187 94.85) (width 0.15) (layer "F.Cu") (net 2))
 (segment (start 112.0925 94.0625) (end 110.63 92.6) (width 0.15) (layer "F.Cu") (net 2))
 (segment (start 110.63 92.6) (end 110.63 93.575) (width 0.15) (layer "F.Cu") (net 2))
 (segment (start 108.84 95.365) (end 104.3 95.365) (width 0.15) (layer "F.Cu") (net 2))
 (segment (start 113.6 95.210187) (end 113.6 95.5275) (width 0.15) (layer "F.Cu") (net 2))
 (segment (start 118.4625 96.545) (end 116.910658 96.545) (width 0.15) (layer "F.Cu") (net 2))
 (segment (start 110.63 93.575) (end 108.84 95.365) (width 0.15) (layer "F.Cu") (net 2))
 (segment (start 112.915 94.0625) (end 112.0925 94.0625) (width 0.15) (layer "F.Cu") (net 2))
 (segment (start 116.910658 96.545) (end 115.215658 94.85) (width 0.15) (layer "F.Cu") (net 2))
 (segment (start 113.960187 94.85) (end 113.6 95.210187) (width 0.15) (layer "F.Cu") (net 2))
 (segment (start 112.915 94.0625) (end 112.915 94.525187) (width 0.15) (layer "F.Cu") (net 2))
 (segment (start 103.224999 94.725001) (end 103.224999 96.829999) (width 0.15) (layer "F.Cu") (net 5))
 (segment (start 103.224999 96.829999) (end 104.3 97.905) (width 0.15) (layer "F.Cu") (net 5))
 (segment (start 115.4425 94.0625) (end 114.8 94.0625) (width 0.15) (layer "F.Cu") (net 5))
 (segment (start 114.13749 93.39999) (end 114.8 94.0625) (width 0.15) (layer "F.Cu") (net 5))
 (segment (start 112.67999 93.39999) (end 114.13749 93.39999) (width 0.15) (layer "F.Cu") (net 5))
 (segment (start 109.36 92.75) (end 109.07 93.04) (width 0.15) (layer "F.Cu") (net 5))
 (segment (start 118.4625 95.895) (end 117.275 95.895) (width 0.15) (layer "F.Cu") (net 5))
 (segment (start 109.36 93.575) (end 108.645001 94.289999) (width 0.15) (layer "F.Cu") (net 5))
 (segment (start 109.36 92.6) (end 109.36 93.575) (width 0.15) (layer "F.Cu") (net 5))
 (segment (start 109.36 92.6) (end 109.36 92.75) (width 0.15) (layer "F.Cu") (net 5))
 (segment (start 109.36 92.6) (end 109.36 91.625) (width 0.15) (layer "F.Cu") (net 5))
 (segment (start 109.36 91.625) (end 109.58501 91.39999) (width 0.15) (layer "F.Cu") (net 5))
 (segment (start 117.275 95.895) (end 115.4425 94.0625) (width 0.15) (layer "F.Cu") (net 5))
 (segment (start 110.937852 91.39999) (end 112.21499 92.677128) (width 0.15) (layer "F.Cu") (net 5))
 (segment (start 112.21499 92.677128) (end 112.21499 92.93499) (width 0.15) (layer "F.Cu") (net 5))
 (segment (start 112.21499 92.93499) (end 112.67999 93.39999) (width 0.15) (layer "F.Cu") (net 5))
 (segment (start 103.660001 94.289999) (end 103.224999 94.725001) (width 0.15) (layer "F.Cu") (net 5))
 (segment (start 108.645001 94.289999) (end 103.660001 94.289999) (width 0.15) (layer "F.Cu") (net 5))
 (segment (start 109.58501 91.39999) (end 110.937852 91.39999) (width 0.15) (layer "F.Cu") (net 5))
 (segment (start 130.275 96.875) (end 131.2 95.95) (width 0.15) (layer "F.Cu") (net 17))
 (segment (start 131.2 95.95) (end 131.2 95.1) (width 0.15) (layer "F.Cu") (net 17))
 (segment (start 130.55 95.1) (end 130.55 95.95) (width 0.15) (layer "F.Cu") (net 18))
 (segment (start 130.55 95.95) (end 130.275 96.225) (width 0.15) (layer "F.Cu") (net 18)))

